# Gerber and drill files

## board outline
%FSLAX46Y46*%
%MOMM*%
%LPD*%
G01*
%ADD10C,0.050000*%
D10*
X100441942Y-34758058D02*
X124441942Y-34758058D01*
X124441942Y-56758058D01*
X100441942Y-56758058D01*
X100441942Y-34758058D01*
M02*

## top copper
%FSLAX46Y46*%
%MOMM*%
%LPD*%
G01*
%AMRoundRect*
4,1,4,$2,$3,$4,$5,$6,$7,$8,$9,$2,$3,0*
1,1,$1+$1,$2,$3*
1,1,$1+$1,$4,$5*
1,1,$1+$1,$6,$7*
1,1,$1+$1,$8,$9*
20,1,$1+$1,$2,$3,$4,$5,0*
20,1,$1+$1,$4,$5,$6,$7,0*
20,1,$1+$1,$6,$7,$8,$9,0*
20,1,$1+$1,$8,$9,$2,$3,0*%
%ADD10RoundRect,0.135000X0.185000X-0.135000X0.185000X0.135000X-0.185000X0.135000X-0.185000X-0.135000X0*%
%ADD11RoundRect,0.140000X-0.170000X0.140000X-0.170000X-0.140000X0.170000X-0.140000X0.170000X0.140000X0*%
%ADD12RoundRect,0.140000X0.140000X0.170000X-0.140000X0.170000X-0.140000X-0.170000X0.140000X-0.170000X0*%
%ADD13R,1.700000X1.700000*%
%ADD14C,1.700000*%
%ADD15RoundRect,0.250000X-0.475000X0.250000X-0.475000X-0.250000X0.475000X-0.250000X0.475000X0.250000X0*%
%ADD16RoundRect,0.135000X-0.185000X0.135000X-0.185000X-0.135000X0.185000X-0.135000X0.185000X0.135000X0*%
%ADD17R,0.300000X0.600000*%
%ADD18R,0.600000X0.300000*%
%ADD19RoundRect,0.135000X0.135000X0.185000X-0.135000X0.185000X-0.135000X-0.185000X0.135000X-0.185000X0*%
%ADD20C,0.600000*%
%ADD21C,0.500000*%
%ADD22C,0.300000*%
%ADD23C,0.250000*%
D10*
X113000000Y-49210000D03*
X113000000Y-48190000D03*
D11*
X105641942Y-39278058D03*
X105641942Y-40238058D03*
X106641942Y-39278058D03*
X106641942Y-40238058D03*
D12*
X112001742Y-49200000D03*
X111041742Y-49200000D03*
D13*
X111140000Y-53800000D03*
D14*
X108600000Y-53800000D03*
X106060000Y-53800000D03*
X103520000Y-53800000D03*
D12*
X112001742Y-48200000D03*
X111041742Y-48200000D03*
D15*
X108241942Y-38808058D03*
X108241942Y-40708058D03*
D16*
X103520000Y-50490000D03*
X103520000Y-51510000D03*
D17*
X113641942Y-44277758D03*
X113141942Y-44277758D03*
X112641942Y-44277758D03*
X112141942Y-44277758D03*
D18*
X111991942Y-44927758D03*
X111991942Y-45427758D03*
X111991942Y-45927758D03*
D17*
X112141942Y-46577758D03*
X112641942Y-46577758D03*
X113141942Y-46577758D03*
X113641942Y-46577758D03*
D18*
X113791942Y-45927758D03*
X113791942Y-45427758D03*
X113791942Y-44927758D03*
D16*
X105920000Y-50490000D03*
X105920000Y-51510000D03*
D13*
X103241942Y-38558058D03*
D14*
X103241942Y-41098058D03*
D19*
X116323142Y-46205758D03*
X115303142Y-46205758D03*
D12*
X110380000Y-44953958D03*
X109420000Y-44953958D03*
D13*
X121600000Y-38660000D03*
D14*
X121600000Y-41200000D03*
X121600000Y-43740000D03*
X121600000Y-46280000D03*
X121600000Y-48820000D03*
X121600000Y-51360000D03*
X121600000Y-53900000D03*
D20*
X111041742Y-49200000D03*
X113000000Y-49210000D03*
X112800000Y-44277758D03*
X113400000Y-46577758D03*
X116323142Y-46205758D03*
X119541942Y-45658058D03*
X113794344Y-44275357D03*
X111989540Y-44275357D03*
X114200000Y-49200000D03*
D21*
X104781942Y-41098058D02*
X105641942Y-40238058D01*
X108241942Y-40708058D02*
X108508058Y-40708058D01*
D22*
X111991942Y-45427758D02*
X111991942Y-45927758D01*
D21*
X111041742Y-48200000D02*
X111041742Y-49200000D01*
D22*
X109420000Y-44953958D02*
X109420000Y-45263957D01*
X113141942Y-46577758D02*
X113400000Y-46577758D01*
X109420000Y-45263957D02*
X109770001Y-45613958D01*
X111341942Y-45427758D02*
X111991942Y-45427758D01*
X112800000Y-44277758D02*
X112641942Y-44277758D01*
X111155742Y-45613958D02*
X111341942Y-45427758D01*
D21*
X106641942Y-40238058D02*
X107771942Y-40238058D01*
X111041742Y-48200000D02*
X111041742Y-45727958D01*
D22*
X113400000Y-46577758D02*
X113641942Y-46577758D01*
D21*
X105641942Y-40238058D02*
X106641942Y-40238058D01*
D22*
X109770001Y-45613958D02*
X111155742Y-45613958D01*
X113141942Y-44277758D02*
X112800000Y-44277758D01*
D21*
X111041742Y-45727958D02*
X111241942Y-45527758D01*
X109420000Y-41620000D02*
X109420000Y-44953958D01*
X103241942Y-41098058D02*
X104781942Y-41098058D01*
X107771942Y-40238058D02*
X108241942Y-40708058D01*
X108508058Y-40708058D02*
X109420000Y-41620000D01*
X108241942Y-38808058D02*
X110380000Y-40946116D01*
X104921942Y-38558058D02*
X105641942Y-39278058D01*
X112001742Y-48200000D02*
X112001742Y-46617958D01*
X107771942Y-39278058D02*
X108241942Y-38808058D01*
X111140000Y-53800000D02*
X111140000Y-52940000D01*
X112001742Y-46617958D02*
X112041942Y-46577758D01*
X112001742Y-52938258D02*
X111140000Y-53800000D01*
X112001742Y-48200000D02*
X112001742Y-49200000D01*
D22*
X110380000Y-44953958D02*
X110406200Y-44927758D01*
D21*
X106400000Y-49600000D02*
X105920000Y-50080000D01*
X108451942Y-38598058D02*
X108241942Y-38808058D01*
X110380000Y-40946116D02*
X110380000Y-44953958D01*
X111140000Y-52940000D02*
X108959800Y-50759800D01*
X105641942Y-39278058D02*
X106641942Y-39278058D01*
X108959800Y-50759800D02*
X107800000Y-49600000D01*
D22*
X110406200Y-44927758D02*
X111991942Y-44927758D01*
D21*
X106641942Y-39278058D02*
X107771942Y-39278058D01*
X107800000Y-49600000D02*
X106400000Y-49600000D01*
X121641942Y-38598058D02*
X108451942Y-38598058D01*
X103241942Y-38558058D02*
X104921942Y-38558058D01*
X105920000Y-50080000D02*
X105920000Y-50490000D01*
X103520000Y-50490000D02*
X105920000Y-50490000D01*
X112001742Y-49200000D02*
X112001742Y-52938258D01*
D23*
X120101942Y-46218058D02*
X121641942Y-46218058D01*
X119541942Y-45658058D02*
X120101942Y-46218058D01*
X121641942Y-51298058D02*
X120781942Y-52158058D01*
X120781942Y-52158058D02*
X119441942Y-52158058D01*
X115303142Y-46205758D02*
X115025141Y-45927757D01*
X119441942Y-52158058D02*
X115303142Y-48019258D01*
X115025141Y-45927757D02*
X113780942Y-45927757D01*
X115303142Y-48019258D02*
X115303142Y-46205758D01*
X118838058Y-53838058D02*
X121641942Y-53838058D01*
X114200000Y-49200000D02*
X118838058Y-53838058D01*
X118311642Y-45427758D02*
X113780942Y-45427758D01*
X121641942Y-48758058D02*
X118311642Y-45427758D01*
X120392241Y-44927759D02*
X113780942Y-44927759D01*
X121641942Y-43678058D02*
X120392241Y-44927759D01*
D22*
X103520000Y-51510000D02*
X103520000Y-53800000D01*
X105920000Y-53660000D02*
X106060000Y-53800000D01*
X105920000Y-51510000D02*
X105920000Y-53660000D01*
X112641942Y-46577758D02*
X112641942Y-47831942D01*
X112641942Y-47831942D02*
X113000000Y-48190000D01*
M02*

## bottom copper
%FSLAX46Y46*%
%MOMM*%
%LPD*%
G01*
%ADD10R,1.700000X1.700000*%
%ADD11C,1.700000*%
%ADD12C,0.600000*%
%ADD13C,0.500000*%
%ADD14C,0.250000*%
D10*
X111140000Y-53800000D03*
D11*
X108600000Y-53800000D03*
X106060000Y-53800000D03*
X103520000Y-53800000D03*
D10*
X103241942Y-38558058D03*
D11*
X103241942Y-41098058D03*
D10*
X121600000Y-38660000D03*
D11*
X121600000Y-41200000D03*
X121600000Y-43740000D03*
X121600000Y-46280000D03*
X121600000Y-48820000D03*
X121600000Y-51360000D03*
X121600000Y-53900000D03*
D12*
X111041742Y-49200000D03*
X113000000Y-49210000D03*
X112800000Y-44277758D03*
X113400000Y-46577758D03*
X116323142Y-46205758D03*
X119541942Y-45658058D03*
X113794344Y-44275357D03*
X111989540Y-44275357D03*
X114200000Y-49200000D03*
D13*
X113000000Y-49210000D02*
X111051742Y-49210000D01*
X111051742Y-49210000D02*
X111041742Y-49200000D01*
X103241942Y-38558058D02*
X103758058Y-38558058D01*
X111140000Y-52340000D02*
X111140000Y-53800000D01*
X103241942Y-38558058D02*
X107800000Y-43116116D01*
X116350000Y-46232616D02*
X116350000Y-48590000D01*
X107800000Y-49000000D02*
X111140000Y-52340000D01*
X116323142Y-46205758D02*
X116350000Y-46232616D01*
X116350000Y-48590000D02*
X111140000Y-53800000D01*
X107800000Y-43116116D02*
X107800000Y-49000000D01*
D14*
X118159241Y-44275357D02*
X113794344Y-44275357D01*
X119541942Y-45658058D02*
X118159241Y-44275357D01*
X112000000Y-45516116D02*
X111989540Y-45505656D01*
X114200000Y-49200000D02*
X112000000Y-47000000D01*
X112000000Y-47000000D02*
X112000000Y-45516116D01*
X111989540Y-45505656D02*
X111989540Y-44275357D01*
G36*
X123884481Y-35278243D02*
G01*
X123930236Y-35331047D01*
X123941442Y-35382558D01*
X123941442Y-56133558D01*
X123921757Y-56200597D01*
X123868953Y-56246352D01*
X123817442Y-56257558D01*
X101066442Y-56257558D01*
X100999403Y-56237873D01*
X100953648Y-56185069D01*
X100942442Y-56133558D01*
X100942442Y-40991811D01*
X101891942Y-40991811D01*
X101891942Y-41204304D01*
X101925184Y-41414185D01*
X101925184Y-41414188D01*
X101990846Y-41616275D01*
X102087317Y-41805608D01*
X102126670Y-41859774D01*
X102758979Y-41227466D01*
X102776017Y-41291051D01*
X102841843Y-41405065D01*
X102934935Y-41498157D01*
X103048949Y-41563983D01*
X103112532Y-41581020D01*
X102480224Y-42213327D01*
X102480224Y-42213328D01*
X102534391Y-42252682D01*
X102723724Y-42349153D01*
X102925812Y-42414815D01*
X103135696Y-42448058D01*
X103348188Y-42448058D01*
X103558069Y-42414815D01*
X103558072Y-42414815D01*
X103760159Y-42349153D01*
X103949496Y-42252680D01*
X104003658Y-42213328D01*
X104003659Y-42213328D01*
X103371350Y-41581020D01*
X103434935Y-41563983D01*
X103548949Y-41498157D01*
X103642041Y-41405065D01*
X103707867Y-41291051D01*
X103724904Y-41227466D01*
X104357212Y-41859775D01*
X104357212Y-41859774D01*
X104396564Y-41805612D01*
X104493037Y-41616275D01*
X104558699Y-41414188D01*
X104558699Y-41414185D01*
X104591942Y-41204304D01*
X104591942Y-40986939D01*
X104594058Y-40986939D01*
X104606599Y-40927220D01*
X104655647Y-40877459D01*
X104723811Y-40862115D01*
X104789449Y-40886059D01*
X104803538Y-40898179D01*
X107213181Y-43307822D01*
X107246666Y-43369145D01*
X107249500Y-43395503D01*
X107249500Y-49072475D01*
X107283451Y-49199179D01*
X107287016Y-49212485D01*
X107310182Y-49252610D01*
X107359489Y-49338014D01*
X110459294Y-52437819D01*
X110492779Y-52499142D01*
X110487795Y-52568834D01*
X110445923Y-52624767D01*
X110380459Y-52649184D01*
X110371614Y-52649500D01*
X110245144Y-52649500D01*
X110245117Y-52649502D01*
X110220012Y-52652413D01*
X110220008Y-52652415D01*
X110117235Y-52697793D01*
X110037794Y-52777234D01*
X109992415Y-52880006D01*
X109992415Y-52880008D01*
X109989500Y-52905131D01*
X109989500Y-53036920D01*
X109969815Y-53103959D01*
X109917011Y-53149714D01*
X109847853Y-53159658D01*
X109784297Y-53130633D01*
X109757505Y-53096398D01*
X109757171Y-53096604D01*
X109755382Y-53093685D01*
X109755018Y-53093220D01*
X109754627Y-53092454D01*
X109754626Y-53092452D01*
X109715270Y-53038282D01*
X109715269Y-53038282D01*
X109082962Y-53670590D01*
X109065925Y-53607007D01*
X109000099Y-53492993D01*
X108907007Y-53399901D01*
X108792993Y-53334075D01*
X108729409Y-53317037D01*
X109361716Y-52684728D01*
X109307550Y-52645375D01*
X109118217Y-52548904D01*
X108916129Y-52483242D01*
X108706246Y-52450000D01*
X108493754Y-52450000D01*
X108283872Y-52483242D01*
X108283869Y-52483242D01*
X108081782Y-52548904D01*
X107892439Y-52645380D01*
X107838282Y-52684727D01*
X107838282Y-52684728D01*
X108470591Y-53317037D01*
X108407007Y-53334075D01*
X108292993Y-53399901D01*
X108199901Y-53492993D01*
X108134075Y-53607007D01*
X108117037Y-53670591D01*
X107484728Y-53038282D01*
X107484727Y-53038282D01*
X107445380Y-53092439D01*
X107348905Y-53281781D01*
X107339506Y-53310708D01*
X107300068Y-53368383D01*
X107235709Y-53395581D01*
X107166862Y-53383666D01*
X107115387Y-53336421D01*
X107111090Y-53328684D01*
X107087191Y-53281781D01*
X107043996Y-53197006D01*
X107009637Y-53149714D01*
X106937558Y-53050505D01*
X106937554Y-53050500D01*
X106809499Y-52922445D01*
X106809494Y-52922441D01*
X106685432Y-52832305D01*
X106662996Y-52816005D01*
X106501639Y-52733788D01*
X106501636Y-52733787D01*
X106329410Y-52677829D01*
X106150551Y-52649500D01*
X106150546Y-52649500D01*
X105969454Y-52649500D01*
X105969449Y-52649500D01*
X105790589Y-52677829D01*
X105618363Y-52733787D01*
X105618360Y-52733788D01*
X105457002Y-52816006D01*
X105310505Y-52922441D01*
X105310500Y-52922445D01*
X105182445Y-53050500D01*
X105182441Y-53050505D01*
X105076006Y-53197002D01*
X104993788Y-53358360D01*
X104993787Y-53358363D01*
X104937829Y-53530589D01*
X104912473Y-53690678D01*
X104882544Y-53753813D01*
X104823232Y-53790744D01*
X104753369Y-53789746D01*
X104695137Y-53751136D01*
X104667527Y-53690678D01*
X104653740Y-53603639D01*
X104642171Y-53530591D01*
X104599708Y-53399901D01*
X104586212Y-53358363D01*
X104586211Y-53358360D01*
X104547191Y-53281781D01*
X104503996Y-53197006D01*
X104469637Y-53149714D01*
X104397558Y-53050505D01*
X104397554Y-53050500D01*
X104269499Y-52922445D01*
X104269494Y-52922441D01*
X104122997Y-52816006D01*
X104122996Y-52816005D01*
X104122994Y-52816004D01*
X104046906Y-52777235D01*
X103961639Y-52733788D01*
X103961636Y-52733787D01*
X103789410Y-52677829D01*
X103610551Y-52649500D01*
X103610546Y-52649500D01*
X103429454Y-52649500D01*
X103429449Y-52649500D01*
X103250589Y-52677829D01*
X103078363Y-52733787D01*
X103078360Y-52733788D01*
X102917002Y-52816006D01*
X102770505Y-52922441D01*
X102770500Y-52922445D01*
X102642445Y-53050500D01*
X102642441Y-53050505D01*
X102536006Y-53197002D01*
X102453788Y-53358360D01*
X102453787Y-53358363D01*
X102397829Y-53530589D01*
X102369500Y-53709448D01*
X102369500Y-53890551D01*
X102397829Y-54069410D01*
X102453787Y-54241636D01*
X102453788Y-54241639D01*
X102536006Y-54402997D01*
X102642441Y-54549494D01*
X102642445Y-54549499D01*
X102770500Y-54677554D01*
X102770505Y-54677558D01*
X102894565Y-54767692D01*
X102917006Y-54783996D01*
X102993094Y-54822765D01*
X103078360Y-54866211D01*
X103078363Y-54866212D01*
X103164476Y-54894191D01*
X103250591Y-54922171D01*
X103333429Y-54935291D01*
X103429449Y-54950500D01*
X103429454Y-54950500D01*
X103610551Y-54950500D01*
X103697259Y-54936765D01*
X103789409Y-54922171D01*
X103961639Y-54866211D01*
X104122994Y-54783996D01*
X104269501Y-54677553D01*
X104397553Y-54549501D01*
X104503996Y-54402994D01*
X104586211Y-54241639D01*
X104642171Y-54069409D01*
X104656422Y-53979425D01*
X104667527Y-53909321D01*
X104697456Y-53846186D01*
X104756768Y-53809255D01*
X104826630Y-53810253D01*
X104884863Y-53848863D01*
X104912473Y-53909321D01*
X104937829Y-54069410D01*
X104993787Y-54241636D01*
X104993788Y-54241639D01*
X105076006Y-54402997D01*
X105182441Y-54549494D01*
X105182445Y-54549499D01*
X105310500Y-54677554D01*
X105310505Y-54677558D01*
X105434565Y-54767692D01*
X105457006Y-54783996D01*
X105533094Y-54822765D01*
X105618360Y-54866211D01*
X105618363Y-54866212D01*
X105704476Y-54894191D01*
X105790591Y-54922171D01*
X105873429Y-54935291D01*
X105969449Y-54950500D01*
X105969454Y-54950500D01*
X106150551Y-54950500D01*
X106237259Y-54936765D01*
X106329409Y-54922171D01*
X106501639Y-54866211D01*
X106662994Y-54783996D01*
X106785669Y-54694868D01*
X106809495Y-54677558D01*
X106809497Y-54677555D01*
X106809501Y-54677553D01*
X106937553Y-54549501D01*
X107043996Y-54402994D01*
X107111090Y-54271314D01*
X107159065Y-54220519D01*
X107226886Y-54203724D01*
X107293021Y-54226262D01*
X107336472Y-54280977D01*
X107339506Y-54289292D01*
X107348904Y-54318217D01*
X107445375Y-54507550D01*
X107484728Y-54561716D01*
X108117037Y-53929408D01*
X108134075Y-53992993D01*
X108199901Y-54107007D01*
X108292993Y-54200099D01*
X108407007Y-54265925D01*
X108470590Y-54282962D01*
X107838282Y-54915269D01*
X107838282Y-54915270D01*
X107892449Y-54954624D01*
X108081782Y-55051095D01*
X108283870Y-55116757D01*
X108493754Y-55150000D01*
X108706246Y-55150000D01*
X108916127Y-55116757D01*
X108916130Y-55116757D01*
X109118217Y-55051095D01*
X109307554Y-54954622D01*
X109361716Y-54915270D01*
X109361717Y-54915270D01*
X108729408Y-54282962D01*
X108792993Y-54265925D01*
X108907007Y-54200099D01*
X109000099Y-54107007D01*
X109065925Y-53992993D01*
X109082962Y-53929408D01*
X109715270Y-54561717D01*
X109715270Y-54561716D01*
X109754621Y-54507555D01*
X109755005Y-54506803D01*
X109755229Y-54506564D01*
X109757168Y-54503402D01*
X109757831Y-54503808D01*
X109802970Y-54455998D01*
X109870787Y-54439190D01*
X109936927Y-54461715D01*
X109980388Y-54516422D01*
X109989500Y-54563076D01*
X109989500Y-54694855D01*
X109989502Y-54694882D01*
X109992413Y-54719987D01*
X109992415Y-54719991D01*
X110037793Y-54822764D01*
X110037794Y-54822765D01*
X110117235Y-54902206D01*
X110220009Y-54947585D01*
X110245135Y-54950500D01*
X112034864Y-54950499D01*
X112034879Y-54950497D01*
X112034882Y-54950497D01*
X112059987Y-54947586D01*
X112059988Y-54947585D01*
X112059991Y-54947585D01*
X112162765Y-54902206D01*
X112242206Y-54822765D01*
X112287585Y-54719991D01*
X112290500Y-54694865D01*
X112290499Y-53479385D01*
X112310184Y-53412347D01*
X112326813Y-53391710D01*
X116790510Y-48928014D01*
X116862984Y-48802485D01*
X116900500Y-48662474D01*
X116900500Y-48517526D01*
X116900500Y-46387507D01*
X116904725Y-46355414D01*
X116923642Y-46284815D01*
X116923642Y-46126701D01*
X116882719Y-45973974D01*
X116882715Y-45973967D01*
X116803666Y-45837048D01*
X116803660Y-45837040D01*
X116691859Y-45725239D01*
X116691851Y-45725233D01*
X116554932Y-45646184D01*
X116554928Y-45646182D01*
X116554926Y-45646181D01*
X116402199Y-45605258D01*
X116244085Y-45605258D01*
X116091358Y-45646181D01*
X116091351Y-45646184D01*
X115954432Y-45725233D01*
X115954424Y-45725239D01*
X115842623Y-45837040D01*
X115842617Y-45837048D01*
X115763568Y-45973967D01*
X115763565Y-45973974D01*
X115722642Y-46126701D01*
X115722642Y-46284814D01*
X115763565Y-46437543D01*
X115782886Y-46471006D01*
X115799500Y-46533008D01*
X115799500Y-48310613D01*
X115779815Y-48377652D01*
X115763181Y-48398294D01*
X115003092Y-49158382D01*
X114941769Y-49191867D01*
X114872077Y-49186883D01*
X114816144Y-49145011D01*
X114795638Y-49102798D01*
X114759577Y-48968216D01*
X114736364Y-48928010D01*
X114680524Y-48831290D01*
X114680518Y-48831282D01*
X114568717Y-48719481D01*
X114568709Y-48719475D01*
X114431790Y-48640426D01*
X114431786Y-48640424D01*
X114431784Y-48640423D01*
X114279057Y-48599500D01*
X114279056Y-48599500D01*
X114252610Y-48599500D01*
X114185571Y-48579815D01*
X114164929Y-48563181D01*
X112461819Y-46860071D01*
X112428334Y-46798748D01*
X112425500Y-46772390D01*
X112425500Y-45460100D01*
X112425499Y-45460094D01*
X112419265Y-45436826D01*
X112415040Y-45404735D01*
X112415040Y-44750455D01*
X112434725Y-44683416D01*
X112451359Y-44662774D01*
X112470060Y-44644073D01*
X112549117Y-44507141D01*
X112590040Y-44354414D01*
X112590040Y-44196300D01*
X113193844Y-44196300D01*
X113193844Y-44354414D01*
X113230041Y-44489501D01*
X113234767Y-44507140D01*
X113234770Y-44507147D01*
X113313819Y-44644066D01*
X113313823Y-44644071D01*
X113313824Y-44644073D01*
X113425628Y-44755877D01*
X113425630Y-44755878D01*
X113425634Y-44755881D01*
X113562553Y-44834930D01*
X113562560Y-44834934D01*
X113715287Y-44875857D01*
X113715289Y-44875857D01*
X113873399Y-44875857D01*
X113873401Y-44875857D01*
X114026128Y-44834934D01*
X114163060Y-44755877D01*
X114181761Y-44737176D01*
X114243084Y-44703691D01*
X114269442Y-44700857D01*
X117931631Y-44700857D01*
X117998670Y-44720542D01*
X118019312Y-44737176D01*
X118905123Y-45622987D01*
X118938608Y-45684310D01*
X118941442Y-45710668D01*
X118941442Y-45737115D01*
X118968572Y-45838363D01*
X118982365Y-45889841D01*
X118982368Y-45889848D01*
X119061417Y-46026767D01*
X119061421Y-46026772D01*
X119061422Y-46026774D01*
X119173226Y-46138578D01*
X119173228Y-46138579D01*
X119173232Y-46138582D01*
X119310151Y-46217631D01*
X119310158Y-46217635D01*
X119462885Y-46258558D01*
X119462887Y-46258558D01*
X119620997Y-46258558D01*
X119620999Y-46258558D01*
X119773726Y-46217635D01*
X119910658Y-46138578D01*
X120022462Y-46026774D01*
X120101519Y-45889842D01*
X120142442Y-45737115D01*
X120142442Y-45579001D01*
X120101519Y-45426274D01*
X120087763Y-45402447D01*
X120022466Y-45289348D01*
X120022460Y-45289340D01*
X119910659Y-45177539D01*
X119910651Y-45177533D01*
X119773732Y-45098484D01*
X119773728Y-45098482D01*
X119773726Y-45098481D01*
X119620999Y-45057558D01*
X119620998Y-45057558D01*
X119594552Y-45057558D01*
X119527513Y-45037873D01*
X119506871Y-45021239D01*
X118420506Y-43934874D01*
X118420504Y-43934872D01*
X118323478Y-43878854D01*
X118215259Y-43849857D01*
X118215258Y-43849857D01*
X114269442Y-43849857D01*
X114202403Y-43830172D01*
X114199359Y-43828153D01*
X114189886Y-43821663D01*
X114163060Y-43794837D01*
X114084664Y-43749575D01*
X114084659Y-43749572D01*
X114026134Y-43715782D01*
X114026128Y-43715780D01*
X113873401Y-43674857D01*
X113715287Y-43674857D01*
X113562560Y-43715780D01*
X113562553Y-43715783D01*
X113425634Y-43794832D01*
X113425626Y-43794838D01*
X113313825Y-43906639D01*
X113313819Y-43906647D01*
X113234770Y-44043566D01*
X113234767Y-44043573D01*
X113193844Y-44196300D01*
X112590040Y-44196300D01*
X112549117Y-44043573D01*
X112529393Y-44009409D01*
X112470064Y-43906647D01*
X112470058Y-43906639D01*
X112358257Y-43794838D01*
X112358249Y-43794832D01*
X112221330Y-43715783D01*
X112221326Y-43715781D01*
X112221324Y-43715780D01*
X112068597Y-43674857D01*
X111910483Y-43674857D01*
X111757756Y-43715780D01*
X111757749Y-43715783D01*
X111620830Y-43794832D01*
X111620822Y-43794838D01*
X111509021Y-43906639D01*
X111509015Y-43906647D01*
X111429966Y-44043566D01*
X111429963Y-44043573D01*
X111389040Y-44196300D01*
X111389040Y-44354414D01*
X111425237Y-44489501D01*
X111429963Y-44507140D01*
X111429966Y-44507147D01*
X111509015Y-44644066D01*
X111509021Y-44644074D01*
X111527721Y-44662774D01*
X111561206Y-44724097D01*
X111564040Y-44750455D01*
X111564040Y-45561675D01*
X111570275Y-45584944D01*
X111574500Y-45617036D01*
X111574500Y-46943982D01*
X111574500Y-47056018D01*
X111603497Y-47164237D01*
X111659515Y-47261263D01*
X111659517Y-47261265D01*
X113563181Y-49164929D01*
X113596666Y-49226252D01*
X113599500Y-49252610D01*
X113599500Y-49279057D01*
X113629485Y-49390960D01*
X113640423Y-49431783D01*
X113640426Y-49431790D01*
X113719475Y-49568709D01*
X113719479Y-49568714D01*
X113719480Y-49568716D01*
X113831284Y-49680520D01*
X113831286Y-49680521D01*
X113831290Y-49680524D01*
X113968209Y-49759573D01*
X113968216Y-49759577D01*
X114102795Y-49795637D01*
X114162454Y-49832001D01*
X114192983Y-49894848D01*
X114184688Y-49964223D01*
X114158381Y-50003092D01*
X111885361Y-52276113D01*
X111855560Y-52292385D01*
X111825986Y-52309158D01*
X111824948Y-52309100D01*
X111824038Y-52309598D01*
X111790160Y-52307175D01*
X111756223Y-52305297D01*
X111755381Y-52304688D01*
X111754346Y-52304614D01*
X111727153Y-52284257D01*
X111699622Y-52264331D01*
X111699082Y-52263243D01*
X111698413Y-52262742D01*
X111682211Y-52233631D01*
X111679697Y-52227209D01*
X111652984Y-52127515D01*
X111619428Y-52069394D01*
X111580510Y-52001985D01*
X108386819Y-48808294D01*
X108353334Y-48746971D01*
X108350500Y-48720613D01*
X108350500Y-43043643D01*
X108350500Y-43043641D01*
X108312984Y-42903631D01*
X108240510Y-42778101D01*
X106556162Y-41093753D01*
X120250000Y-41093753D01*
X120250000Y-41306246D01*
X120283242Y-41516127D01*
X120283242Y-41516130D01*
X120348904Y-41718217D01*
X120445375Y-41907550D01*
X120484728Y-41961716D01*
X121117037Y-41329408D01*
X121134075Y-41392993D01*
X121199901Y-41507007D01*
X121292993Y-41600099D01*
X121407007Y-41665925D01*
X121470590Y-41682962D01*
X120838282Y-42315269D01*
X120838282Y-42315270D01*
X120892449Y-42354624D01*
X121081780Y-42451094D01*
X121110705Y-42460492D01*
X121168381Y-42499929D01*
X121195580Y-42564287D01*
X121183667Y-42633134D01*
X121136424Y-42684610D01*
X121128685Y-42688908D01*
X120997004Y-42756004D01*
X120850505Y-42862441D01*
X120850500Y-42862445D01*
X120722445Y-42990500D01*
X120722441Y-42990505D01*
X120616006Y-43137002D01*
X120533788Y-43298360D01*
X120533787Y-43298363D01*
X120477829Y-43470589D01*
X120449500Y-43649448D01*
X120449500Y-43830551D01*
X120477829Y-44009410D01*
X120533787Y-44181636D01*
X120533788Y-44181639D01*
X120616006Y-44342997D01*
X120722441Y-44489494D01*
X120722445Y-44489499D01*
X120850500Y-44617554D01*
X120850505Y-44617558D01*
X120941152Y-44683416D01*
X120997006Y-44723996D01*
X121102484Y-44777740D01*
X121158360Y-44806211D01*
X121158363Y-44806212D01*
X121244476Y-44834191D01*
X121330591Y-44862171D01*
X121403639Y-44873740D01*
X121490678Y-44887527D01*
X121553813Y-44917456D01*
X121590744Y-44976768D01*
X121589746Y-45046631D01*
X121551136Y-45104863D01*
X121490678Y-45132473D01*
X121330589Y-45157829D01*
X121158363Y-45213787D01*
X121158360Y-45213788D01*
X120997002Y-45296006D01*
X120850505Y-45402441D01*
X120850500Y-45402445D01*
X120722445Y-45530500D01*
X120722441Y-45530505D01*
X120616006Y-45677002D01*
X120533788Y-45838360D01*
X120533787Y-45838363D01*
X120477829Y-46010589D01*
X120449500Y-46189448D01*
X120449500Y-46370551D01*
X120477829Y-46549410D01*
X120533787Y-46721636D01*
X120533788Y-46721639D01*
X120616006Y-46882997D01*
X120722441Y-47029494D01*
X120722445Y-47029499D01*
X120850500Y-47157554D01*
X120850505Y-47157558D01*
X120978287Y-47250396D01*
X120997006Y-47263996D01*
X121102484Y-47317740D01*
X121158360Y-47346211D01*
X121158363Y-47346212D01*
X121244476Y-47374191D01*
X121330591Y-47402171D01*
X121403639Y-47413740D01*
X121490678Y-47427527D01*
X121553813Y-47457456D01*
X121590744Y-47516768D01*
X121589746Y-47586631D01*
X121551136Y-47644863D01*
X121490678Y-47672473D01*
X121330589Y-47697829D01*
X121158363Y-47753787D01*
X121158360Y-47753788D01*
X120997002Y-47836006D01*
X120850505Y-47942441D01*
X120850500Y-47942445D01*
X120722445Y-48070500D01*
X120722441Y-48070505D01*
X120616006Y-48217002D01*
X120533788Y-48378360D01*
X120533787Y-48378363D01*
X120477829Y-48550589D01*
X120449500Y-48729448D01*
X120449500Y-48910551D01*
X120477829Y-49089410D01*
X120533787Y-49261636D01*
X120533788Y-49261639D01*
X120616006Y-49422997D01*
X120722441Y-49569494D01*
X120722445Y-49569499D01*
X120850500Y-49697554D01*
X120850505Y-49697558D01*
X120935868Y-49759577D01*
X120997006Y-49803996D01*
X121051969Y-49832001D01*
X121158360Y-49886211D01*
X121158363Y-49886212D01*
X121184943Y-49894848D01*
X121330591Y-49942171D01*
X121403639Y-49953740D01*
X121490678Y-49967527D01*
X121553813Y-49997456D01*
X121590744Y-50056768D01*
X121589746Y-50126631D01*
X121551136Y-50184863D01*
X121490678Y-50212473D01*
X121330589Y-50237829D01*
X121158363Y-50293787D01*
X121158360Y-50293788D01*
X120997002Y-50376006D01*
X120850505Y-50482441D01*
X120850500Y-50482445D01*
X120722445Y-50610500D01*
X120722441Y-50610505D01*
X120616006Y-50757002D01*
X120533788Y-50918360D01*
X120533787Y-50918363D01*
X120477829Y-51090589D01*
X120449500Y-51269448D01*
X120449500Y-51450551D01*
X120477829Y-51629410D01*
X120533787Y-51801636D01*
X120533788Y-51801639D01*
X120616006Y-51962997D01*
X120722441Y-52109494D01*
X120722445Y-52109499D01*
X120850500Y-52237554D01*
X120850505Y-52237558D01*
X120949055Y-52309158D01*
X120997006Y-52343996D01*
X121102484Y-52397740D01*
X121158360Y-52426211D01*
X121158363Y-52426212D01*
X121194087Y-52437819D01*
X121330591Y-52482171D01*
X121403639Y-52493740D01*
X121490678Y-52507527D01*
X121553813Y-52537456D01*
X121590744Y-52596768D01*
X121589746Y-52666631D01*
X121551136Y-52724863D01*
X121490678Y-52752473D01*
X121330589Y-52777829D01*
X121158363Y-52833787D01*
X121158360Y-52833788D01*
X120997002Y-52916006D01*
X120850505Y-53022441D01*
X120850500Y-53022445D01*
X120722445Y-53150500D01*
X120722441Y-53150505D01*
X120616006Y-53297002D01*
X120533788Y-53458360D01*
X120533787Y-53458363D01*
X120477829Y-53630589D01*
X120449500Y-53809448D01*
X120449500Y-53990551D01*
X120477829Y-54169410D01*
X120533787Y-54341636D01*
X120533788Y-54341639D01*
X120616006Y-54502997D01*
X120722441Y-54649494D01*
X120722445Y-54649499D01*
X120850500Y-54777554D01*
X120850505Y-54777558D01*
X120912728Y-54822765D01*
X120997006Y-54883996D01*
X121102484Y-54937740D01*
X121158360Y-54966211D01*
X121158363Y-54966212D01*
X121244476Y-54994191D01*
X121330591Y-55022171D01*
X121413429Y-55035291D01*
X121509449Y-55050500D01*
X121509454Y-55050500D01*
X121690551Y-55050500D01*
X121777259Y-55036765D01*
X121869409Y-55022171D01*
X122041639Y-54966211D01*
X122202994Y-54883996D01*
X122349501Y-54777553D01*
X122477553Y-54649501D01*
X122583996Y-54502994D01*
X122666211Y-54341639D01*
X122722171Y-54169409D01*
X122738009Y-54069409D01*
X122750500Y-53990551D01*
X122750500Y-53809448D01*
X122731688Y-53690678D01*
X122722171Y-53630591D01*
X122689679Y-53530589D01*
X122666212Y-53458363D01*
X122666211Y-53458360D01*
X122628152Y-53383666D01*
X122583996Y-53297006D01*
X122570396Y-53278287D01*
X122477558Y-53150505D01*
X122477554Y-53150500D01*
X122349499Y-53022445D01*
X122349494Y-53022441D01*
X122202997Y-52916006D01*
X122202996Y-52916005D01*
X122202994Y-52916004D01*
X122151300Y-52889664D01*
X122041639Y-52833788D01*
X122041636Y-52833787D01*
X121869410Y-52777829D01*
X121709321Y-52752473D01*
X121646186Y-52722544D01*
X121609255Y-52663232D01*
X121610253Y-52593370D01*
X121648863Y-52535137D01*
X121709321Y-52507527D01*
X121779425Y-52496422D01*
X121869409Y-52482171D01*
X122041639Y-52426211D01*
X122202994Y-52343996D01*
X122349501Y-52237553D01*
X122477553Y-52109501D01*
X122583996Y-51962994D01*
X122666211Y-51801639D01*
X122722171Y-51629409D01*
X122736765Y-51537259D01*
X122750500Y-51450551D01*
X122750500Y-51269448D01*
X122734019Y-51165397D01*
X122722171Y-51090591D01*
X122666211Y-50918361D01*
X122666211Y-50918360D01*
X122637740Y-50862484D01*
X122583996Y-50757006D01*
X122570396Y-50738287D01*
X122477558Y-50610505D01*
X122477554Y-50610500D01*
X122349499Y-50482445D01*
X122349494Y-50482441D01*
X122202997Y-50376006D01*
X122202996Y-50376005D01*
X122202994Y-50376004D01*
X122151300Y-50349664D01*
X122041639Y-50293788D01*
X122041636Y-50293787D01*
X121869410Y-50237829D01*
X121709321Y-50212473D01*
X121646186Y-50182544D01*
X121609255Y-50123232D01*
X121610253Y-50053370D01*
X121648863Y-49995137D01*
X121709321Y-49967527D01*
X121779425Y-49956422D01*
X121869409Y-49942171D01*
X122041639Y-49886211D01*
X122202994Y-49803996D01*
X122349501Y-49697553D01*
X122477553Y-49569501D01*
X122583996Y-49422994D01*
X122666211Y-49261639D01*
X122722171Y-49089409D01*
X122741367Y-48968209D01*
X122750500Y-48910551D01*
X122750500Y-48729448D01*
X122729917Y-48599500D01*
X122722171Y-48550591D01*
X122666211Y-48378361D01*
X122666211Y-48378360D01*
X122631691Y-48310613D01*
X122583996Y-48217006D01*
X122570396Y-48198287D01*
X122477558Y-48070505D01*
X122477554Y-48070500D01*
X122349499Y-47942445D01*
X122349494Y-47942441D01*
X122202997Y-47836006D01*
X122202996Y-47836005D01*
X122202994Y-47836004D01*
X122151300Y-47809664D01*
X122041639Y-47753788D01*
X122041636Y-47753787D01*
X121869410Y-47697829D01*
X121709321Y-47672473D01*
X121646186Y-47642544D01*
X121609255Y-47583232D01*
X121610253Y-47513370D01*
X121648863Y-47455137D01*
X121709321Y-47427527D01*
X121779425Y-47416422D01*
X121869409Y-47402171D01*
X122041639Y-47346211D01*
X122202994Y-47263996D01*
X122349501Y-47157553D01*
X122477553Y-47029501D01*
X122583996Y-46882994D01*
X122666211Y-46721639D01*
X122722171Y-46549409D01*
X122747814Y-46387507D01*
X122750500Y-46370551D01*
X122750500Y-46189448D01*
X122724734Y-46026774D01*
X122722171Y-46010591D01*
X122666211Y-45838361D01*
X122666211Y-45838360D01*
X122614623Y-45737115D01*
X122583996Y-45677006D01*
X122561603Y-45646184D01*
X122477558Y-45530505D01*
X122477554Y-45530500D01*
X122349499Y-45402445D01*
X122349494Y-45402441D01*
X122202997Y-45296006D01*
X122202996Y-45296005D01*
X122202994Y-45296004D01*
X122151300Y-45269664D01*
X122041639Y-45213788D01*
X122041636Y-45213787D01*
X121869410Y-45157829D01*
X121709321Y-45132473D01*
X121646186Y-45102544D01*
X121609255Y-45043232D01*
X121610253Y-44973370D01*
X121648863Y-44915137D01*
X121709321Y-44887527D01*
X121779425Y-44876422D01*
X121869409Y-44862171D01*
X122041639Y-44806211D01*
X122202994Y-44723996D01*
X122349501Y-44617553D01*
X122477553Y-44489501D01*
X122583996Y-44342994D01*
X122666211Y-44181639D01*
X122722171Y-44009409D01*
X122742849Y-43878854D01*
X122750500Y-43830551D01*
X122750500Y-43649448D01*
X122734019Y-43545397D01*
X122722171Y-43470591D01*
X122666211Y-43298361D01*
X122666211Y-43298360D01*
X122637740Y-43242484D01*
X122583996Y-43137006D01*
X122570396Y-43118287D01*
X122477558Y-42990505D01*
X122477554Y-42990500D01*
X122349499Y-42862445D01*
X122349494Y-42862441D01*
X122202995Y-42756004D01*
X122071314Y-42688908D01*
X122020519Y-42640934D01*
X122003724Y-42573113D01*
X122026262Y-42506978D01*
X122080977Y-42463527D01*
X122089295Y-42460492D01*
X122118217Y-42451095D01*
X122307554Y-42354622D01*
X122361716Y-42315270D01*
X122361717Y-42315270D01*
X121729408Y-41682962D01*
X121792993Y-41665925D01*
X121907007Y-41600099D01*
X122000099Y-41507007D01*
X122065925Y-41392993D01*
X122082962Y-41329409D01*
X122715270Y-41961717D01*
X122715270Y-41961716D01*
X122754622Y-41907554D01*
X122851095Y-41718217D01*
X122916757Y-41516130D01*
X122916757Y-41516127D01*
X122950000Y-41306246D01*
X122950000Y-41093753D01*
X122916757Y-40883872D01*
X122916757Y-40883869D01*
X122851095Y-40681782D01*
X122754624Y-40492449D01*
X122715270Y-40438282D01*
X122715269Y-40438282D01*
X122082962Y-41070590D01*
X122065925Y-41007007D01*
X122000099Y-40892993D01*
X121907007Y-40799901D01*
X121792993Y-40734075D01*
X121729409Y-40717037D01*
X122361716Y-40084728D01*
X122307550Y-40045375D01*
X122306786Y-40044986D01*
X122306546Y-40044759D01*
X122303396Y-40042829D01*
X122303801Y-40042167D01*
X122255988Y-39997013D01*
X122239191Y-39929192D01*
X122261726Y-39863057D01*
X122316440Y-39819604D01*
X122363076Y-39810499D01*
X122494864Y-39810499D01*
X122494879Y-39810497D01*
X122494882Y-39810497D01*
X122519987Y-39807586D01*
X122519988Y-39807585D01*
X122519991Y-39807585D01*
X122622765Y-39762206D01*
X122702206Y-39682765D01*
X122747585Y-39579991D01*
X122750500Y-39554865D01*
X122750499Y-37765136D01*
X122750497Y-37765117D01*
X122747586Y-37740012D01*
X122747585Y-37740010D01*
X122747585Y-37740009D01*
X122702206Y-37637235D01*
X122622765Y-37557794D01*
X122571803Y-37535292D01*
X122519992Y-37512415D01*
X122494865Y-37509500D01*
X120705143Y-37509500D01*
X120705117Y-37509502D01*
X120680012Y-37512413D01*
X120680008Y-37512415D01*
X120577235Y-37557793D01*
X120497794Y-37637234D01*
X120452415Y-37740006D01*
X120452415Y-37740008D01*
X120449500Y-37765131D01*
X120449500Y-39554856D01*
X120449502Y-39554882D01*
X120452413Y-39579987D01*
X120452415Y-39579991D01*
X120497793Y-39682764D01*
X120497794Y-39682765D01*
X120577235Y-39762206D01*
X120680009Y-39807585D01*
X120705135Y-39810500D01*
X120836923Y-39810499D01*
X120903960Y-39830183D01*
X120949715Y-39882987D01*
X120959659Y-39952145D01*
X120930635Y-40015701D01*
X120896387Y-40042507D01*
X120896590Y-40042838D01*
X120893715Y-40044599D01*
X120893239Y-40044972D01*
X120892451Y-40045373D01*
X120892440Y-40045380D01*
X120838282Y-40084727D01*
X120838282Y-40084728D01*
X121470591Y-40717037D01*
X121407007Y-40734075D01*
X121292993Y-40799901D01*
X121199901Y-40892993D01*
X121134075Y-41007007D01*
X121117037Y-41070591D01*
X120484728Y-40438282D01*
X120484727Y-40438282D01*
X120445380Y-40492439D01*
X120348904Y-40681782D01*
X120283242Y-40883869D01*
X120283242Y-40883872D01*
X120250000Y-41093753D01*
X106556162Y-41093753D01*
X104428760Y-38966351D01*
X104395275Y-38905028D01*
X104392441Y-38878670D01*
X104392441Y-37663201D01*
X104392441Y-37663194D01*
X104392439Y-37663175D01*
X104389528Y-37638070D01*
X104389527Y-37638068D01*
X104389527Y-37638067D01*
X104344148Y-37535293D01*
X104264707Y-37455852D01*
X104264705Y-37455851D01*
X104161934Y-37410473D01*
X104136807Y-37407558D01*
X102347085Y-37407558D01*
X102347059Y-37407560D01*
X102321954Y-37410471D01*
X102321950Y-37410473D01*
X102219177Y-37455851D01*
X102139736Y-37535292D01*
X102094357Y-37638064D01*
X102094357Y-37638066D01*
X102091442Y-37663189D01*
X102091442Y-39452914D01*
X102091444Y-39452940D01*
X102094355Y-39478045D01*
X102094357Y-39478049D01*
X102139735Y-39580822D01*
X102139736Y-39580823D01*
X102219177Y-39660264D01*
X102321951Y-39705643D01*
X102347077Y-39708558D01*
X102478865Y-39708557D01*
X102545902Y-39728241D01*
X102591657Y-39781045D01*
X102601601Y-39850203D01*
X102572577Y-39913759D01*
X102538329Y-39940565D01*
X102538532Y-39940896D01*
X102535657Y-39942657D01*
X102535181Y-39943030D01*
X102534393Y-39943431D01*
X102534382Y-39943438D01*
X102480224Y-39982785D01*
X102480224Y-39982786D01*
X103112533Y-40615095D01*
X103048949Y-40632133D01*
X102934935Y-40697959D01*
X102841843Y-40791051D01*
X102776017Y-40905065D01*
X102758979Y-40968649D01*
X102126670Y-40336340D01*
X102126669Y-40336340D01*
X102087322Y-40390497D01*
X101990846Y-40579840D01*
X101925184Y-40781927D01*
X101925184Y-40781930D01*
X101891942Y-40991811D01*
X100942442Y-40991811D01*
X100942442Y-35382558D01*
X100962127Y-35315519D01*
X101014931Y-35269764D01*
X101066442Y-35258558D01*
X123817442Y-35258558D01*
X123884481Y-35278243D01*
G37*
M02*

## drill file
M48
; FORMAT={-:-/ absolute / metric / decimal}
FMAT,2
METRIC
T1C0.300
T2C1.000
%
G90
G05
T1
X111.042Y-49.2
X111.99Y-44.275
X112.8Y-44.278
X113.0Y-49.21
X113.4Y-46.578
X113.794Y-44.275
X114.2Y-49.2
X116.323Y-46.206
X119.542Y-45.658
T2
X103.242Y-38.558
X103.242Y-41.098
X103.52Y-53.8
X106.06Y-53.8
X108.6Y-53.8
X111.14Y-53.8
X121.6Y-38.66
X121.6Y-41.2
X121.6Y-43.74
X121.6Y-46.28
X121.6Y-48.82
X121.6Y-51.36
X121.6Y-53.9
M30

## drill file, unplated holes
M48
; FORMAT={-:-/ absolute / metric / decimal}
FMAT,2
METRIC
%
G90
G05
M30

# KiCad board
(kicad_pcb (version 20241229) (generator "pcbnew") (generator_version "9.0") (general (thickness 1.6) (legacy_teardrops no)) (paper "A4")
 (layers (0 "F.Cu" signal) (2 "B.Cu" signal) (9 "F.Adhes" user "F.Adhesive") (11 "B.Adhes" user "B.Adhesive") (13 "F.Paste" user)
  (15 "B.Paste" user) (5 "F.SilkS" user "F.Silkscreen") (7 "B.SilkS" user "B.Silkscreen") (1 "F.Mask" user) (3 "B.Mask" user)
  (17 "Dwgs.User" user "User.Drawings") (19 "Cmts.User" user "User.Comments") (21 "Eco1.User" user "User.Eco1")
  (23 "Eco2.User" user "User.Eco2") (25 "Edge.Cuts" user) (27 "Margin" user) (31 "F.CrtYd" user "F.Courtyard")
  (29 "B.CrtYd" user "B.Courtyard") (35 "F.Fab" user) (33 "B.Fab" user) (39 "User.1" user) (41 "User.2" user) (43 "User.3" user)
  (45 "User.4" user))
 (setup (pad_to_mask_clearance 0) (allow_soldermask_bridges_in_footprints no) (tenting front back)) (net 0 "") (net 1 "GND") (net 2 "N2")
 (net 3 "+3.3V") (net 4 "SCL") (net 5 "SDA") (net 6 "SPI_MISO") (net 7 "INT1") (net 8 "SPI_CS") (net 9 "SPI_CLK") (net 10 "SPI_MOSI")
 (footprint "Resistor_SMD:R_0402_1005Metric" (layer "F.Cu") (at 113 48.7 90)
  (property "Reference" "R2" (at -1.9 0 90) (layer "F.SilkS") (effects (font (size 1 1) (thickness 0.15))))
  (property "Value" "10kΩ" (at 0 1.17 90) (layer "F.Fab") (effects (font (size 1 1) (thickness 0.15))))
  (pad "1" smd roundrect (at -0.51 0 90) (size 0.54 0.64) (layers "F.Cu" "F.Mask" "F.Paste") (roundrect_rratio 0.25) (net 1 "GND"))
  (pad "2" smd roundrect (at 0.51 0 90) (size 0.54 0.64) (layers "F.Cu" "F.Mask" "F.Paste") (roundrect_rratio 0.25) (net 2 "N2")))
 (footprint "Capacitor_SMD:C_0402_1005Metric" (layer "F.Cu") (at 105.641942 39.758058 -90)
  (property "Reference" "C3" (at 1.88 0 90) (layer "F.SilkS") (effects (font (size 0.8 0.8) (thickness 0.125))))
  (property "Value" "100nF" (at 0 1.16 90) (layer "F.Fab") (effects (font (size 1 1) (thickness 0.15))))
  (pad "1" smd roundrect (at -0.48 0 270) (size 0.56 0.62) (layers "F.Cu" "F.Mask" "F.Paste") (roundrect_rratio 0.25) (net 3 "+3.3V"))
  (pad "2" smd roundrect (at 0.48 0 270) (size 0.56 0.62) (layers "F.Cu" "F.Mask" "F.Paste") (roundrect_rratio 0.25) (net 1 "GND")))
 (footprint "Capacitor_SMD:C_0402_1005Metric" (layer "F.Cu") (at 106.641942 39.758058 -90)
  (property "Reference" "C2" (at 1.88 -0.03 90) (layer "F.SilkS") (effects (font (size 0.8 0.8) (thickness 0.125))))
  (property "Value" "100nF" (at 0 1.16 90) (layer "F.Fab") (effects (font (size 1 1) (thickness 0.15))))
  (pad "1" smd roundrect (at -0.48 0 270) (size 0.56 0.62) (layers "F.Cu" "F.Mask" "F.Paste") (roundrect_rratio 0.25) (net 3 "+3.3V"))
  (pad "2" smd roundrect (at 0.48 0 270) (size 0.56 0.62) (layers "F.Cu" "F.Mask" "F.Paste") (roundrect_rratio 0.25) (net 1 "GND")))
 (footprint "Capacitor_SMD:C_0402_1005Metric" (layer "F.Cu") (at 111.521742 49.2 180)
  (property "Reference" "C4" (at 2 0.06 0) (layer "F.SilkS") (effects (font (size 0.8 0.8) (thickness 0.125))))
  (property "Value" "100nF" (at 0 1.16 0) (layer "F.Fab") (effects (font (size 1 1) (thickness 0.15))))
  (pad "1" smd roundrect (at -0.48 0 180) (size 0.56 0.62) (layers "F.Cu" "F.Mask" "F.Paste") (roundrect_rratio 0.25) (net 3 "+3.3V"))
  (pad "2" smd roundrect (at 0.48 0 180) (size 0.56 0.62) (layers "F.Cu" "F.Mask" "F.Paste") (roundrect_rratio 0.25) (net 1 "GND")))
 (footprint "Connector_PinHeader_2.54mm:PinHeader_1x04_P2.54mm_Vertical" (layer "F.Cu") (at 111.14 53.8 -90)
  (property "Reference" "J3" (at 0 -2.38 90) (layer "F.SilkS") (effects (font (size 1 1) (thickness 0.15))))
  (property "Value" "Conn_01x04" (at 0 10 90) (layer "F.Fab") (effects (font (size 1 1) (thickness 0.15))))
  (pad "1" thru_hole rect (at 0 0 270) (size 1.7 1.7) (drill 1) (layers "*.Cu" "*.Mask") (remove_unused_layers no) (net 3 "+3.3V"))
  (pad "2" thru_hole circle (at 0 2.54 270) (size 1.7 1.7) (drill 1) (layers "*.Cu" "*.Mask") (remove_unused_layers no) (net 1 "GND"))
  (pad "3" thru_hole circle (at 0 5.08 270) (size 1.7 1.7) (drill 1) (layers "*.Cu" "*.Mask") (remove_unused_layers no) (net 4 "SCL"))
  (pad "4" thru_hole circle (at 0 7.62 270) (size 1.7 1.7) (drill 1) (layers "*.Cu" "*.Mask") (remove_unused_layers no) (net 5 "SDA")))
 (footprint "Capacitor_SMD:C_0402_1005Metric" (layer "F.Cu") (at 111.521742 48.2 180)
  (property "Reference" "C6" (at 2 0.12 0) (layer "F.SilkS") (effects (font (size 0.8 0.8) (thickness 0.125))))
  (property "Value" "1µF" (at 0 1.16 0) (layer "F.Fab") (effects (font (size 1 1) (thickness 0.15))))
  (pad "1" smd roundrect (at -0.48 0 180) (size 0.56 0.62) (layers "F.Cu" "F.Mask" "F.Paste") (roundrect_rratio 0.25) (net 3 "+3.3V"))
  (pad "2" smd roundrect (at 0.48 0 180) (size 0.56 0.62) (layers "F.Cu" "F.Mask" "F.Paste") (roundrect_rratio 0.25) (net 1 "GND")))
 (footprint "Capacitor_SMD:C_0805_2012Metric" (layer "F.Cu") (at 108.241942 39.758058 -90)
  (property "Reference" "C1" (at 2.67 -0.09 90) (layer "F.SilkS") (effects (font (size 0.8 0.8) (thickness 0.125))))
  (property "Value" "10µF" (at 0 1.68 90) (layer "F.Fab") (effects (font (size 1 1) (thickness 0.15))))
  (pad "1" smd roundrect (at -0.95 0 270) (size 1 1.45) (layers "F.Cu" "F.Mask" "F.Paste") (roundrect_rratio 0.25) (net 3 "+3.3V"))
  (pad "2" smd roundrect (at 0.95 0 270) (size 1 1.45) (layers "F.Cu" "F.Mask" "F.Paste") (roundrect_rratio 0.25) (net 1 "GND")))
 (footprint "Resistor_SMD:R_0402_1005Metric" (layer "F.Cu") (at 103.52 51 -90)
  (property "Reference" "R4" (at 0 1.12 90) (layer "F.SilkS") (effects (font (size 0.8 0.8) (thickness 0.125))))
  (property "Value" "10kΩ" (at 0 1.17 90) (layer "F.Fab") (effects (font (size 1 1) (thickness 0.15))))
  (pad "1" smd roundrect (at -0.51 0 270) (size 0.54 0.64) (layers "F.Cu" "F.Mask" "F.Paste") (roundrect_rratio 0.25) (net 3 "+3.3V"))
  (pad "2" smd roundrect (at 0.51 0 270) (size 0.54 0.64) (layers "F.Cu" "F.Mask" "F.Paste") (roundrect_rratio 0.25) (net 5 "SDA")))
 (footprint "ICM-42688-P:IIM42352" (layer "F.Cu") (at 112.891942 45.427758 -90)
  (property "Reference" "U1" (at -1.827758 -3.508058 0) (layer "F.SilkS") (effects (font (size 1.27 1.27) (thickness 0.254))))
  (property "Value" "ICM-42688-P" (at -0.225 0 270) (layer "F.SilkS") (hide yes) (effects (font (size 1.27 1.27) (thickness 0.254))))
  (pad "1" smd rect (at -1.15 -0.75) (size 0.3 0.6) (layers "F.Cu" "F.Mask" "F.Paste") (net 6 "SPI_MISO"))
  (pad "2" smd rect (at -1.15 -0.25) (size 0.3 0.6) (layers "F.Cu" "F.Mask" "F.Paste") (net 1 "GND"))
  (pad "3" smd rect (at -1.15 0.25) (size 0.3 0.6) (layers "F.Cu" "F.Mask" "F.Paste") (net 1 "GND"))
  (pad "4" smd rect (at -1.15 0.75) (size 0.3 0.6) (layers "F.Cu" "F.Mask" "F.Paste") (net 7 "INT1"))
  (pad "5" smd rect (at -0.5 0.9 270) (size 0.3 0.6) (layers "F.Cu" "F.Mask" "F.Paste") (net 3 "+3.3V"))
  (pad "6" smd rect (at 0 0.9 270) (size 0.3 0.6) (layers "F.Cu" "F.Mask" "F.Paste") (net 1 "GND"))
  (pad "7" smd rect (at 0.5 0.9 270) (size 0.3 0.6) (layers "F.Cu" "F.Mask" "F.Paste") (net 1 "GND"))
  (pad "8" smd rect (at 1.15 0.75) (size 0.3 0.6) (layers "F.Cu" "F.Mask" "F.Paste") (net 3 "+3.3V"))
  (pad "9" smd rect (at 1.15 0.25) (size 0.3 0.6) (layers "F.Cu" "F.Mask" "F.Paste") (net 2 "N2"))
  (pad "10" smd rect (at 1.15 -0.25) (size 0.3 0.6) (layers "F.Cu" "F.Mask" "F.Paste") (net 1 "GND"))
  (pad "11" smd rect (at 1.15 -0.75) (size 0.3 0.6) (layers "F.Cu" "F.Mask" "F.Paste") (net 1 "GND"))
  (pad "12" smd rect (at 0.5 -0.9 270) (size 0.3 0.6) (layers "F.Cu" "F.Mask" "F.Paste") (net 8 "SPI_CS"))
  (pad "13" smd rect (at 0 -0.9 270) (size 0.3 0.6) (layers "F.Cu" "F.Mask" "F.Paste") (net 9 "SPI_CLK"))
  (pad "14" smd rect (at -0.5 -0.9 270) (size 0.3 0.6) (layers "F.Cu" "F.Mask" "F.Paste") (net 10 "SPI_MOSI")))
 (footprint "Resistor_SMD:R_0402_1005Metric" (layer "F.Cu") (at 105.92 51 -90)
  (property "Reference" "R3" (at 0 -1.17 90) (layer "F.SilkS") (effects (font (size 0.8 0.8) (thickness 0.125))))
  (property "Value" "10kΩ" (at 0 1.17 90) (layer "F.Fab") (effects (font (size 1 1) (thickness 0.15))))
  (pad "1" smd roundrect (at -0.51 0 270) (size 0.54 0.64) (layers "F.Cu" "F.Mask" "F.Paste") (roundrect_rratio 0.25) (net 3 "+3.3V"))
  (pad "2" smd roundrect (at 0.51 0 270) (size 0.54 0.64) (layers "F.Cu" "F.Mask" "F.Paste") (roundrect_rratio 0.25) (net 4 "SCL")))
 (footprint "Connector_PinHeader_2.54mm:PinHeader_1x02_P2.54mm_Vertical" (layer "F.Cu") (at 103.241942 38.558058)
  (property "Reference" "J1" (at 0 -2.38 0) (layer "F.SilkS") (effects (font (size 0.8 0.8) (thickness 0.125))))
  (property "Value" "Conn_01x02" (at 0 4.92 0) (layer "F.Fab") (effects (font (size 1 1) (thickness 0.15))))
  (pad "1" thru_hole rect (at 0 0) (size 1.7 1.7) (drill 1) (layers "*.Cu" "*.Mask") (remove_unused_layers no) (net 3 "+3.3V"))
  (pad "2" thru_hole circle (at 0 2.54) (size 1.7 1.7) (drill 1) (layers "*.Cu" "*.Mask") (remove_unused_layers no) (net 1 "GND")))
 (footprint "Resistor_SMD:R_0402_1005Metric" (layer "F.Cu") (at 115.813142 46.205758 180)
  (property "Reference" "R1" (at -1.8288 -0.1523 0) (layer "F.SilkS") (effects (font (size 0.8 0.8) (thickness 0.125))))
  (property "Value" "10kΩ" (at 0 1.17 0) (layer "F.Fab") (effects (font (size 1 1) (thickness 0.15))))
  (pad "1" smd roundrect (at -0.51 0 180) (size 0.54 0.64) (layers "F.Cu" "F.Mask" "F.Paste") (roundrect_rratio 0.25) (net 3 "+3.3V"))
  (pad "2" smd roundrect (at 0.51 0 180) (size 0.54 0.64) (layers "F.Cu" "F.Mask" "F.Paste") (roundrect_rratio 0.25) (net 8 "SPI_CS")))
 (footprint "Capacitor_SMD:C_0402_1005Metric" (layer "F.Cu") (at 109.9 44.953958 180)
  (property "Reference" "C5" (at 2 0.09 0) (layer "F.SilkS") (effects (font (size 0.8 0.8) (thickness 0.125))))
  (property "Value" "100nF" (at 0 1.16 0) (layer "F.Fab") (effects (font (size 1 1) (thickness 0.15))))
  (pad "1" smd roundrect (at -0.48 0 180) (size 0.56 0.62) (layers "F.Cu" "F.Mask" "F.Paste") (roundrect_rratio 0.25) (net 3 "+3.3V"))
  (pad "2" smd roundrect (at 0.48 0 180) (size 0.56 0.62) (layers "F.Cu" "F.Mask" "F.Paste") (roundrect_rratio 0.25) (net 1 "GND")))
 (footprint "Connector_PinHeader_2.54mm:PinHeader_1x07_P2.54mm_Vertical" (layer "F.Cu") (at 121.6 38.66)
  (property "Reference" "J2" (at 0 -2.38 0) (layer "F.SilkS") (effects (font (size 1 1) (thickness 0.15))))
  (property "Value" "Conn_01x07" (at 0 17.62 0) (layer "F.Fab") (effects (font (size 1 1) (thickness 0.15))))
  (pad "1" thru_hole rect (at 0 0) (size 1.7 1.7) (drill 1) (layers "*.Cu" "*.Mask") (remove_unused_layers no) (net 3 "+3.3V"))
  (pad "2" thru_hole circle (at 0 2.54) (size 1.7 1.7) (drill 1) (layers "*.Cu" "*.Mask") (remove_unused_layers no) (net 1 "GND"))
  (pad "3" thru_hole circle (at 0 5.08) (size 1.7 1.7) (drill 1) (layers "*.Cu" "*.Mask") (remove_unused_layers no) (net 10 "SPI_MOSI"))
  (pad "4" thru_hole circle (at 0 7.62) (size 1.7 1.7) (drill 1) (layers "*.Cu" "*.Mask") (remove_unused_layers no) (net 6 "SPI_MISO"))
  (pad "5" thru_hole circle (at 0 10.16) (size 1.7 1.7) (drill 1) (layers "*.Cu" "*.Mask") (remove_unused_layers no) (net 9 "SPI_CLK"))
  (pad "6" thru_hole circle (at 0 12.7) (size 1.7 1.7) (drill 1) (layers "*.Cu" "*.Mask") (remove_unused_layers no) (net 8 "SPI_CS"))
  (pad "7" thru_hole circle (at 0 15.24) (size 1.7 1.7) (drill 1) (layers "*.Cu" "*.Mask") (remove_unused_layers no) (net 7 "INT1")))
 (gr_rect (start 100.441942 34.758058) (end 124.441942 56.758058) (stroke (width 0.05) (type default)) (fill no) (layer "Edge.Cuts"))
 (segment (start 104.781942 41.098058) (end 105.641942 40.238058) (width 0.5) (layer "F.Cu") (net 1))
 (segment (start 108.241942 40.708058) (end 108.508058 40.708058) (width 0.5) (layer "F.Cu") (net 1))
 (segment (start 111.991942 45.427758) (end 111.991942 45.927758) (width 0.3) (layer "F.Cu") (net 1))
 (segment (start 111.041742 48.2) (end 111.041742 49.2) (width 0.5) (layer "F.Cu") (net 1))
 (segment (start 109.42 44.953958) (end 109.42 45.263957) (width 0.3) (layer "F.Cu") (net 1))
 (segment (start 113.141942 46.577758) (end 113.4 46.577758) (width 0.3) (layer "F.Cu") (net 1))
 (segment (start 109.42 45.263957) (end 109.770001 45.613958) (width 0.3) (layer "F.Cu") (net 1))
 (segment (start 111.341942 45.427758) (end 111.991942 45.427758) (width 0.3) (layer "F.Cu") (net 1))
 (segment (start 112.8 44.277758) (end 112.641942 44.277758) (width 0.3) (layer "F.Cu") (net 1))
 (segment (start 111.155742 45.613958) (end 111.341942 45.427758) (width 0.3) (layer "F.Cu") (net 1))
 (segment (start 106.641942 40.238058) (end 107.771942 40.238058) (width 0.5) (layer "F.Cu") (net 1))
 (segment (start 111.041742 48.2) (end 111.041742 45.727958) (width 0.5) (layer "F.Cu") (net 1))
 (segment (start 113.4 46.577758) (end 113.641942 46.577758) (width 0.3) (layer "F.Cu") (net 1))
 (segment (start 105.641942 40.238058) (end 106.641942 40.238058) (width 0.5) (layer "F.Cu") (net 1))
 (segment (start 109.770001 45.613958) (end 111.155742 45.613958) (width 0.3) (layer "F.Cu") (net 1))
 (segment (start 113.141942 44.277758) (end 112.8 44.277758) (width 0.3) (layer "F.Cu") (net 1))
 (segment (start 111.041742 45.727958) (end 111.241942 45.527758) (width 0.5) (layer "F.Cu") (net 1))
 (segment (start 109.42 41.62) (end 109.42 44.953958) (width 0.5) (layer "F.Cu") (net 1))
 (segment (start 103.241942 41.098058) (end 104.781942 41.098058) (width 0.5) (layer "F.Cu") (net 1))
 (segment (start 107.771942 40.238058) (end 108.241942 40.708058) (width 0.5) (layer "F.Cu") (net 1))
 (segment (start 108.508058 40.708058) (end 109.42 41.62) (width 0.5) (layer "F.Cu") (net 1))
 (via (at 111.041742 49.2) (size 0.6) (drill 0.3) (layers "F.Cu" "B.Cu") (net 1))
 (via (at 113 49.21) (size 0.6) (drill 0.3) (layers "F.Cu" "B.Cu") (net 1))
 (via (at 112.8 44.277758) (size 0.6) (drill 0.3) (layers "F.Cu" "B.Cu") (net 1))
 (via (at 113.4 46.577758) (size 0.6) (drill 0.3) (layers "F.Cu" "B.Cu") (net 1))
 (segment (start 113 49.21) (end 111.051742 49.21) (width 0.5) (layer "B.Cu") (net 1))
 (segment (start 111.051742 49.21) (end 111.041742 49.2) (width 0.5) (layer "B.Cu") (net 1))
 (segment (start 108.241942 38.808058) (end 110.38 40.946116) (width 0.5) (layer "F.Cu") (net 3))
 (segment (start 104.921942 38.558058) (end 105.641942 39.278058) (width 0.5) (layer "F.Cu") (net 3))
 (segment (start 112.001742 48.2) (end 112.001742 46.617958) (width 0.5) (layer "F.Cu") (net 3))
 (segment (start 107.771942 39.278058) (end 108.241942 38.808058) (width 0.5) (layer "F.Cu") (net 3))
 (segment (start 111.14 53.8) (end 111.14 52.94) (width 0.5) (layer "F.Cu") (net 3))
 (segment (start 112.001742 46.617958) (end 112.041942 46.577758) (width 0.5) (layer "F.Cu") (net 3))
 (segment (start 112.001742 52.938258) (end 111.14 53.8) (width 0.5) (layer "F.Cu") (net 3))
 (segment (start 112.001742 48.2) (end 112.001742 49.2) (width 0.5) (layer "F.Cu") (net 3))
 (segment (start 110.38 44.953958) (end 110.4062 44.927758) (width 0.3) (layer "F.Cu") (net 3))
 (segment (start 106.4 49.6) (end 105.92 50.08) (width 0.5) (layer "F.Cu") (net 3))
 (segment (start 108.451942 38.598058) (end 108.241942 38.808058) (width 0.5) (layer "F.Cu") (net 3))
 (segment (start 110.38 40.946116) (end 110.38 44.953958) (width 0.5) (layer "F.Cu") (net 3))
 (segment (start 111.14 52.94) (end 108.9598 50.7598) (width 0.5) (layer "F.Cu") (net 3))
 (segment (start 105.641942 39.278058) (end 106.641942 39.278058) (width 0.5) (layer "F.Cu") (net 3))
 (segment (start 108.9598 50.7598) (end 107.8 49.6) (width 0.5) (layer "F.Cu") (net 3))
 (segment (start 110.4062 44.927758) (end 111.991942 44.927758) (width 0.3) (layer "F.Cu") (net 3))
 (segment (start 106.641942 39.278058) (end 107.771942 39.278058) (width 0.5) (layer "F.Cu") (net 3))
 (segment (start 107.8 49.6) (end 106.4 49.6) (width 0.5) (layer "F.Cu") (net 3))
 (segment (start 121.641942 38.598058) (end 108.451942 38.598058) (width 0.5) (layer "F.Cu") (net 3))
 (segment (start 103.241942 38.558058) (end 104.921942 38.558058) (width 0.5) (layer "F.Cu") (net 3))
 (segment (start 105.92 50.08) (end 105.92 50.49) (width 0.5) (layer "F.Cu") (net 3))
 (segment (start 103.52 50.49) (end 105.92 50.49) (width 0.5) (layer "F.Cu") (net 3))
 (segment (start 112.001742 49.2) (end 112.001742 52.938258) (width 0.5) (layer "F.Cu") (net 3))
 (via (at 116.323142 46.205758) (size 0.6) (drill 0.3) (layers "F.Cu" "B.Cu") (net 3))
 (segment (start 103.241942 38.558058) (end 103.758058 38.558058) (width 0.5) (layer "B.Cu") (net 3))
 (segment (start 111.14 52.34) (end 111.14 53.8) (width 0.5) (layer "B.Cu") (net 3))
 (segment (start 103.241942 38.558058) (end 107.8 43.116116) (width 0.5) (layer "B.Cu") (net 3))
 (segment (start 116.35 46.232616) (end 116.35 48.59) (width 0.5) (layer "B.Cu") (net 3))
 (segment (start 107.8 49) (end 111.14 52.34) (width 0.5) (layer "B.Cu") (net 3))
 (segment (start 116.323142 46.205758) (end 116.35 46.232616) (width 0.5) (layer "B.Cu") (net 3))
 (segment (start 116.35 48.59) (end 111.14 53.8) (width 0.5) (layer "B.Cu") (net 3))
 (segment (start 107.8 43.116116) (end 107.8 49) (width 0.5) (layer "B.Cu") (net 3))
 (segment (start 120.101942 46.218058) (end 121.641942 46.218058) (width 0.25) (layer "F.Cu") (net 6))
 (segment (start 119.541942 45.658058) (end 120.101942 46.218058) (width 0.25) (layer "F.Cu") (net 6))
 (via (at 119.541942 45.658058) (size 0.6) (drill 0.3) (layers "F.Cu" "B.Cu") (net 6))
 (via (at 113.794344 44.275357) (size 0.6) (drill 0.3) (layers "F.Cu" "B.Cu") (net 6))
 (segment (start 118.159241 44.275357) (end 113.794344 44.275357) (width 0.25) (layer "B.Cu") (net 6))
 (segment (start 119.541942 45.658058) (end 118.159241 44.275357) (width 0.25) (layer "B.Cu") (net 6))
 (segment (start 121.641942 51.298058) (end 120.781942 52.158058) (width 0.25) (layer "F.Cu") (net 8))
 (segment (start 120.781942 52.158058) (end 119.441942 52.158058) (width 0.25) (layer "F.Cu") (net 8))
 (segment (start 115.303142 46.205758) (end 115.025141 45.927757) (width 0.25) (layer "F.Cu") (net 8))
 (segment (start 119.441942 52.158058) (end 115.303142 48.019258) (width 0.25) (layer "F.Cu") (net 8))
 (segment (start 115.025141 45.927757) (end 113.780942 45.927757) (width 0.25) (layer "F.Cu") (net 8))
 (segment (start 115.303142 48.019258) (end 115.303142 46.205758) (width 0.25) (layer "F.Cu") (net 8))
 (segment (start 118.838058 53.838058) (end 121.641942 53.838058) (width 0.25) (layer "F.Cu") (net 7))
 (segment (start 114.2 49.2) (end 118.838058 53.838058) (width 0.25) (layer "F.Cu") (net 7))
 (via (at 111.98954 44.275357) (size 0.6) (drill 0.3) (layers "F.Cu" "B.Cu") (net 7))
 (via (at 114.2 49.2) (size 0.6) (drill 0.3) (layers "F.Cu" "B.Cu") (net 7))
 (segment (start 112 45.516116) (end 111.98954 45.505656) (width 0.25) (layer "B.Cu") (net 7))
 (segment (start 114.2 49.2) (end 112 47) (width 0.25) (layer "B.Cu") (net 7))
 (segment (start 112 47) (end 112 45.516116) (width 0.25) (layer "B.Cu") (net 7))
 (segment (start 111.98954 45.505656) (end 111.98954 44.275357) (width 0.25) (layer "B.Cu") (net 7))
 (segment (start 118.311642 45.427758) (end 113.780942 45.427758) (width 0.25) (layer "F.Cu") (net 9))
 (segment (start 121.641942 48.758058) (end 118.311642 45.427758) (width 0.25) (layer "F.Cu") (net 9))
 (segment (start 120.392241 44.927759) (end 113.780942 44.927759) (width 0.25) (layer "F.Cu") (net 10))
 (segment (start 121.641942 43.678058) (end 120.392241 44.927759) (width 0.25) (layer "F.Cu") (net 10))
 (segment (start 103.52 51.51) (end 103.52 53.8) (width 0.3) (layer "F.Cu") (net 5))
 (segment (start 105.92 53.66) (end 106.06 53.8) (width 0.3) (layer "F.Cu") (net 4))
 (segment (start 105.92 51.51) (end 105.92 53.66) (width 0.3) (layer "F.Cu") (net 4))
 (segment (start 112.641942 46.577758) (end 112.641942 47.831942) (width 0.3) (layer "F.Cu") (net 2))
 (segment (start 112.641942 47.831942) (end 113 48.19) (width 0.3) (layer "F.Cu") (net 2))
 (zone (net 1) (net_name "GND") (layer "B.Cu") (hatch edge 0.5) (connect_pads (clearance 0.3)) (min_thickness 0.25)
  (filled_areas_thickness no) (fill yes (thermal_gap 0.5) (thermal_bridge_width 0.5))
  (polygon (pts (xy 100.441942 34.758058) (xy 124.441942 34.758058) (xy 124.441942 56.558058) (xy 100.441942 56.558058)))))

